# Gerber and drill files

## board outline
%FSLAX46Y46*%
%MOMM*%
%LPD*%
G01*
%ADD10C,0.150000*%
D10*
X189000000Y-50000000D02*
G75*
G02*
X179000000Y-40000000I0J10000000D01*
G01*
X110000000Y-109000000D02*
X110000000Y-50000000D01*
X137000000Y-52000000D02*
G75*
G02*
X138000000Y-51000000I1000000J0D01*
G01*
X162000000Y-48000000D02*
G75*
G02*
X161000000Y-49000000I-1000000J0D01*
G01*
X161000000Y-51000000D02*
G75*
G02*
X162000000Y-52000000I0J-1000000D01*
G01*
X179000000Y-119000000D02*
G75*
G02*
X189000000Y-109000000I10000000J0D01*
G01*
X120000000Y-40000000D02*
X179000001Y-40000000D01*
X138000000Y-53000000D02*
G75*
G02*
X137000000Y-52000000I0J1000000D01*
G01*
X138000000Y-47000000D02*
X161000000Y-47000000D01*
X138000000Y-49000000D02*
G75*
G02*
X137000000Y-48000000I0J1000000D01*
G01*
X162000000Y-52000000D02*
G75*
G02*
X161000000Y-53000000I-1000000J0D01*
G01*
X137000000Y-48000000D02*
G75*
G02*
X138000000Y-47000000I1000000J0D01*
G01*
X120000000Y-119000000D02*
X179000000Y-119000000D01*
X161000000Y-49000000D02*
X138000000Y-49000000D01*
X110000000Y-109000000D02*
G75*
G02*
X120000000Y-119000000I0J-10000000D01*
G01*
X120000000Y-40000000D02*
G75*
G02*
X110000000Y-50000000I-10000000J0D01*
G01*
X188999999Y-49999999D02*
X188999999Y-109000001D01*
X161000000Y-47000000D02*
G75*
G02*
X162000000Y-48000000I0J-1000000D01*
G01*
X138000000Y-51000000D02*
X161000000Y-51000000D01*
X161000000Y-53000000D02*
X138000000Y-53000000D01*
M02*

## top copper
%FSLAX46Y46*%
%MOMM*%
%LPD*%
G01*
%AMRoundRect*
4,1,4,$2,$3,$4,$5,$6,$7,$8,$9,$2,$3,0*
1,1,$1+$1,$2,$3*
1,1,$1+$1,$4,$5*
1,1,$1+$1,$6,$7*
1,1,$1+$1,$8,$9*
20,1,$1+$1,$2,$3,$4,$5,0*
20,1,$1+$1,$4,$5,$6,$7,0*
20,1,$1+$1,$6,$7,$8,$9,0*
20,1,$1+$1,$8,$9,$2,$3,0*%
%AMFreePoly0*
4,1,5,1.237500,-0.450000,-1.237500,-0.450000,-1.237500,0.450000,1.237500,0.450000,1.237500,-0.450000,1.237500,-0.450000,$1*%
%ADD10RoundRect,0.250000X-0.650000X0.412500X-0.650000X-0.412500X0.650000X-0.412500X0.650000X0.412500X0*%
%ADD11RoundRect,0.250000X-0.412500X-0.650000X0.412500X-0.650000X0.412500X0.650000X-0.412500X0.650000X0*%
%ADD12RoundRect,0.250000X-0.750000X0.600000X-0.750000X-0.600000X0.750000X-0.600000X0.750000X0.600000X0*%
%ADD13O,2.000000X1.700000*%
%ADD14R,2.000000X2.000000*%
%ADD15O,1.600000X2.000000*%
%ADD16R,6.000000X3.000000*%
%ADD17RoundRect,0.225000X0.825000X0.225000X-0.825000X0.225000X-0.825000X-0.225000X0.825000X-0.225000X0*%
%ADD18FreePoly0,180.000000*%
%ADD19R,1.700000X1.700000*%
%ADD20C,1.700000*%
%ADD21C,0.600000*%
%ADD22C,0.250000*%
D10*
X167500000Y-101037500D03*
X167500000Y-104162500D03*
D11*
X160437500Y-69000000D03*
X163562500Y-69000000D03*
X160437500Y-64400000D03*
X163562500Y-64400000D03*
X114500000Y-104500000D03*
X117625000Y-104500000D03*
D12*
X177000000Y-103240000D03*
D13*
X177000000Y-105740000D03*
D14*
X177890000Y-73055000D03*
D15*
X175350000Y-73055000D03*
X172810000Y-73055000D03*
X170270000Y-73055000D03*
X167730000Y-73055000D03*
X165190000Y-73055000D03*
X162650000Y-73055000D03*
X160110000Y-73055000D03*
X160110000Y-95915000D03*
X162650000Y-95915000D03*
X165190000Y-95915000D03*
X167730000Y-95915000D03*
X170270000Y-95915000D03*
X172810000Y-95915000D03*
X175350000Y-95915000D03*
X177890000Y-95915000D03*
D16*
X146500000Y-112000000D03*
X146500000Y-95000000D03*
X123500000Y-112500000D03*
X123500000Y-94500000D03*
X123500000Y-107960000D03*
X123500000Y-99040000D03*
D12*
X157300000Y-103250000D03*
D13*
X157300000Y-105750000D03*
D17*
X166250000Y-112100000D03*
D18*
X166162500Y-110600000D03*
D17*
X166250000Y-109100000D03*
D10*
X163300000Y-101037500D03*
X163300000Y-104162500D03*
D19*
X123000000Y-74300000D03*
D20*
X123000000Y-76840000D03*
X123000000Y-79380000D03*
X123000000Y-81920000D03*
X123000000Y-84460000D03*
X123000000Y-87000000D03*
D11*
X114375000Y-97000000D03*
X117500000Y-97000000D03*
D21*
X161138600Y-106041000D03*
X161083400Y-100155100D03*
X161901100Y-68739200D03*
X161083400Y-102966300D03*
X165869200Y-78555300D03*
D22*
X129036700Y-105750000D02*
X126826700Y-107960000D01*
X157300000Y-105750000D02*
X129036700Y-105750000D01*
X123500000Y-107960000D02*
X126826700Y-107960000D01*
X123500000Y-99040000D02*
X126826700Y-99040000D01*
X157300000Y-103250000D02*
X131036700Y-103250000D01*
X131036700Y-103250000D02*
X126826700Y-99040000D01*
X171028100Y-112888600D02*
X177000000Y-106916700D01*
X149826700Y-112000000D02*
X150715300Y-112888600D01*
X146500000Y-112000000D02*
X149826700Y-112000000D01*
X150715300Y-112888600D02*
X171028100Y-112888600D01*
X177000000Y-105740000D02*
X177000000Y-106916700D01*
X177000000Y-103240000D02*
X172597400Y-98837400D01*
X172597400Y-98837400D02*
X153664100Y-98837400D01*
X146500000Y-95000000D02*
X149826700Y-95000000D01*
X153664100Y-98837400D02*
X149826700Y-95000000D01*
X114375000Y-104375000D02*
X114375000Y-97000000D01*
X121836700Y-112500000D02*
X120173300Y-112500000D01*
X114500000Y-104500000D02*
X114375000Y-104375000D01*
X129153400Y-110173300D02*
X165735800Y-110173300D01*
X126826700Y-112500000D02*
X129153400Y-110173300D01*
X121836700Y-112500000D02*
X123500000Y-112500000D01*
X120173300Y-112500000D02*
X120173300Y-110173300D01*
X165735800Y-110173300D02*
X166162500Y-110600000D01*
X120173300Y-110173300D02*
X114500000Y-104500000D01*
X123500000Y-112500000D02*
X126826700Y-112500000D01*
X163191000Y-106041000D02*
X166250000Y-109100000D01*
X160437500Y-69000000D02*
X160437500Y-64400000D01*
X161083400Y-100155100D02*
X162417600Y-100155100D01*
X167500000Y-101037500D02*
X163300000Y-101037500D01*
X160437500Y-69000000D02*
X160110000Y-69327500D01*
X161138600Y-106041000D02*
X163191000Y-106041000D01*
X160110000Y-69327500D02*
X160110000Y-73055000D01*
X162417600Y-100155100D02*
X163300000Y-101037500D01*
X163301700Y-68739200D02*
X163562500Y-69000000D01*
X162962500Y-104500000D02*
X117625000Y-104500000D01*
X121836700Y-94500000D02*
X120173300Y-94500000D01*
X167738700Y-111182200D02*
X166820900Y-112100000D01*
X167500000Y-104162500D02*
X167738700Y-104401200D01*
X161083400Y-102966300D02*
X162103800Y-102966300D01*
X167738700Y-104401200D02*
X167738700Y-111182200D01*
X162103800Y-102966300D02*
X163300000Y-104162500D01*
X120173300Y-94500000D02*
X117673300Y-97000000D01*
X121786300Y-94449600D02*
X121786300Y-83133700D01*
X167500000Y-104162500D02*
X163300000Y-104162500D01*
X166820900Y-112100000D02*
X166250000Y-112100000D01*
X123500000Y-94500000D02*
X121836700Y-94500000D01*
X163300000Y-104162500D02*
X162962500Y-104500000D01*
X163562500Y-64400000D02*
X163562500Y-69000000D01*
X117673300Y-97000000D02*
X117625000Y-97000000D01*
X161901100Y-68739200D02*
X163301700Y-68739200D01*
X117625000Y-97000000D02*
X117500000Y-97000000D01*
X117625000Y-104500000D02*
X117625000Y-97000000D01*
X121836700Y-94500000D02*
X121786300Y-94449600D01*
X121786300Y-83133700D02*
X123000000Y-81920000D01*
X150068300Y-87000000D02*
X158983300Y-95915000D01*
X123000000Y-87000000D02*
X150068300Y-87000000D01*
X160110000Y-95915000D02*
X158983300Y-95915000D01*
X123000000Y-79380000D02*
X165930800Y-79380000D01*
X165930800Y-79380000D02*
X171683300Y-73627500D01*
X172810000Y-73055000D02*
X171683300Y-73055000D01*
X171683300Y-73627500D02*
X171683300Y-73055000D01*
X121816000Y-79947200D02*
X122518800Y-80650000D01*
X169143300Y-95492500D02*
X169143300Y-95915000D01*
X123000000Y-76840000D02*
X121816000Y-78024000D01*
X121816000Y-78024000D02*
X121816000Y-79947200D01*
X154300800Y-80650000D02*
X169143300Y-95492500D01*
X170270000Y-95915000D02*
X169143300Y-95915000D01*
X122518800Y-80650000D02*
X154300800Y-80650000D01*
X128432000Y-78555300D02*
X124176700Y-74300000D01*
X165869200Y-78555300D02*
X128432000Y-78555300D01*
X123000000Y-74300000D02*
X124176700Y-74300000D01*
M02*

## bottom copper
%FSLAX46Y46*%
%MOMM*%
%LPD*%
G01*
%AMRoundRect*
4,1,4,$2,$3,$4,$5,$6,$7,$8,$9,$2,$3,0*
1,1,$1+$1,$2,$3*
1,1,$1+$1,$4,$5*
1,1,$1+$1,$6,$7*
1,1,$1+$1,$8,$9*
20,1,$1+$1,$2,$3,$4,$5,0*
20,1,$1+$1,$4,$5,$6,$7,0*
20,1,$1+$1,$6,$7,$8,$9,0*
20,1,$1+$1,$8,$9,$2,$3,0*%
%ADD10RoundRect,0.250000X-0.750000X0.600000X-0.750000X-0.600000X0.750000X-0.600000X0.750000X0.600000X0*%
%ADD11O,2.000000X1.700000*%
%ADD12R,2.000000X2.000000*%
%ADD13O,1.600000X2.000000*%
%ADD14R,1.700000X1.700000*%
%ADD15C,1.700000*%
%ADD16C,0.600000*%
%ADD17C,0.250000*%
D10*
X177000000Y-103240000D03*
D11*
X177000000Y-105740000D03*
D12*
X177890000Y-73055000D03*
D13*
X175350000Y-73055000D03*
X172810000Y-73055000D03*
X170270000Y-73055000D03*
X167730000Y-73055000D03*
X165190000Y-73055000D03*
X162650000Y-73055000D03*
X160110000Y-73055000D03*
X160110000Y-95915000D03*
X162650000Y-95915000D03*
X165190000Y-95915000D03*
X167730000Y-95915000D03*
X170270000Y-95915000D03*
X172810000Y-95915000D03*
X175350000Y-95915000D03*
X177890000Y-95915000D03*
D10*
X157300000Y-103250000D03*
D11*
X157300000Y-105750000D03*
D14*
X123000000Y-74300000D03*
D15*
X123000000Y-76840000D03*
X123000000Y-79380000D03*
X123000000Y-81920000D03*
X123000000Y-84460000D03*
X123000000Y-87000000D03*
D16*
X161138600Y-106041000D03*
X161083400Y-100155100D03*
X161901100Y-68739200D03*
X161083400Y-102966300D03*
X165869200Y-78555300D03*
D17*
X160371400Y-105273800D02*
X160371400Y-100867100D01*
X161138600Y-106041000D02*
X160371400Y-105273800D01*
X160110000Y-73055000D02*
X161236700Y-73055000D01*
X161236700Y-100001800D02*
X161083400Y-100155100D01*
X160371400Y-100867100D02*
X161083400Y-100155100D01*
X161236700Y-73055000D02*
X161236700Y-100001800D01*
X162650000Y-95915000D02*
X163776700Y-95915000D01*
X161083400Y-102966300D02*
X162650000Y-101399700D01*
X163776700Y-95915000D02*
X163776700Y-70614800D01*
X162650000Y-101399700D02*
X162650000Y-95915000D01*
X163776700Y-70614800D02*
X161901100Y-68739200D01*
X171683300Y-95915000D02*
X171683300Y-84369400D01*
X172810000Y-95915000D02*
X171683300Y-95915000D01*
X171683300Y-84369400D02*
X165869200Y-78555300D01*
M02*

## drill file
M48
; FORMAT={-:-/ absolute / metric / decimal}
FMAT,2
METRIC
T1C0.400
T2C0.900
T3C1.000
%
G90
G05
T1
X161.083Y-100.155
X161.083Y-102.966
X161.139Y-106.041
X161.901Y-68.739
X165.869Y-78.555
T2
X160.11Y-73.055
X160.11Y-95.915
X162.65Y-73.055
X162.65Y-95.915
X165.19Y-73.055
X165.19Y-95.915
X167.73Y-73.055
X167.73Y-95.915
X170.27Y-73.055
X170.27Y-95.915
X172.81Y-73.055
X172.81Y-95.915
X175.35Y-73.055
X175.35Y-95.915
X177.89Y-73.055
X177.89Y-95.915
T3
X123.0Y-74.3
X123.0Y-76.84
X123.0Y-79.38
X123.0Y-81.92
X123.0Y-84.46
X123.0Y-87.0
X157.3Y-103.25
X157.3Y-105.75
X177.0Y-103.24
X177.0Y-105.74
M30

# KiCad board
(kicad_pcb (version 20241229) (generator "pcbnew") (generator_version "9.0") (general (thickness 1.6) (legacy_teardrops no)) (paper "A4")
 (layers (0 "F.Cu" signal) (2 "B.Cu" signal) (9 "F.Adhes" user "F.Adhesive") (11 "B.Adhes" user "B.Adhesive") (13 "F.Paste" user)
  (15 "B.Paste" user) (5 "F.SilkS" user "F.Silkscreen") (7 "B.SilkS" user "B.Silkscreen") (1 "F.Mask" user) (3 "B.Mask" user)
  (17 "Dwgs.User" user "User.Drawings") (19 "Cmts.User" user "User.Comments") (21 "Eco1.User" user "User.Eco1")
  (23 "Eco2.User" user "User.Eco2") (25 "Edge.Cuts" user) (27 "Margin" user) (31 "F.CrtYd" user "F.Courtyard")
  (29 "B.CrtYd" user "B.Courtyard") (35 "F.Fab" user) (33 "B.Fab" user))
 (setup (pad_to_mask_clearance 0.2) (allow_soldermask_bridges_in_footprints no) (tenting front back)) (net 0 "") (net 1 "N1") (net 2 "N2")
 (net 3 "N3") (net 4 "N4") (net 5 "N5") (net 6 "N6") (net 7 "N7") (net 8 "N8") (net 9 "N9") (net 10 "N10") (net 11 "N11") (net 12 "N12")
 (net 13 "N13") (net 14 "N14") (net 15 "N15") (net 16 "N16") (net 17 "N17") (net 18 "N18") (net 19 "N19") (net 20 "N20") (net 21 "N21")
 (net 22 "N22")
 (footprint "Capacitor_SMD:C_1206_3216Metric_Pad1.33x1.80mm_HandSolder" (layer "F.Cu") (at 167.5 102.6 -90)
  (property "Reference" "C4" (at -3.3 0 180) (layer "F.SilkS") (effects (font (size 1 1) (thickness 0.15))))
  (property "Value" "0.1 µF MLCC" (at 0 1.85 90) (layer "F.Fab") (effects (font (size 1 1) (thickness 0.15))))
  (pad "1" smd roundrect (at -1.5625 0 270) (size 1.325 1.8) (layers "F.Cu" "F.Mask" "F.Paste") (roundrect_rratio 0.188679) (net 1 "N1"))
  (pad "2" smd roundrect (at 1.5625 0 270) (size 1.325 1.8) (layers "F.Cu" "F.Mask" "F.Paste") (roundrect_rratio 0.188679) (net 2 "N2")))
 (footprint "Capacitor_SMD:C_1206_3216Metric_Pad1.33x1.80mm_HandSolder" (layer "F.Cu") (at 162 69)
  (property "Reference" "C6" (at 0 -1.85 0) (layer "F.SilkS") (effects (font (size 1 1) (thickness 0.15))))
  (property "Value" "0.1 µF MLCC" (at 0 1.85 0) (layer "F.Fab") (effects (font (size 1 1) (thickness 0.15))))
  (pad "1" smd roundrect (at -1.5625 0) (size 1.325 1.8) (layers "F.Cu" "F.Mask" "F.Paste") (roundrect_rratio 0.188679) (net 1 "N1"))
  (pad "2" smd roundrect (at 1.5625 0) (size 1.325 1.8) (layers "F.Cu" "F.Mask" "F.Paste") (roundrect_rratio 0.188679) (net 2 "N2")))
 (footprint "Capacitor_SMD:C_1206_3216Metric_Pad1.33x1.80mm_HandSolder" (layer "F.Cu") (at 162 64.4)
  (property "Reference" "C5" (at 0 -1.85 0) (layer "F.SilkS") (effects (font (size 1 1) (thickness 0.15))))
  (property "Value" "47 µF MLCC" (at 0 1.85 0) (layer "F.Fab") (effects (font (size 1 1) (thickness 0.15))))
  (pad "1" smd roundrect (at -1.5625 0) (size 1.325 1.8) (layers "F.Cu" "F.Mask" "F.Paste") (roundrect_rratio 0.188679) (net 1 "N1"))
  (pad "2" smd roundrect (at 1.5625 0) (size 1.325 1.8) (layers "F.Cu" "F.Mask" "F.Paste") (roundrect_rratio 0.188679) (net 2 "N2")))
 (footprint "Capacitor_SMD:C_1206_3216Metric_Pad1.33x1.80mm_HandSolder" (layer "F.Cu") (at 116.0625 104.5)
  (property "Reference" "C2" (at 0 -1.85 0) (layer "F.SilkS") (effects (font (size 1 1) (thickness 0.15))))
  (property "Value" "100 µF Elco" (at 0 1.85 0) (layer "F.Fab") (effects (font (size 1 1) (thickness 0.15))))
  (pad "1" smd roundrect (at -1.5625 0) (size 1.325 1.8) (layers "F.Cu" "F.Mask" "F.Paste") (roundrect_rratio 0.188679) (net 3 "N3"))
  (pad "2" smd roundrect (at 1.5625 0) (size 1.325 1.8) (layers "F.Cu" "F.Mask" "F.Paste") (roundrect_rratio 0.188679) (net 2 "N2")))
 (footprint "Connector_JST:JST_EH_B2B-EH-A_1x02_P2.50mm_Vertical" (layer "F.Cu") (at 177 103.24 -90)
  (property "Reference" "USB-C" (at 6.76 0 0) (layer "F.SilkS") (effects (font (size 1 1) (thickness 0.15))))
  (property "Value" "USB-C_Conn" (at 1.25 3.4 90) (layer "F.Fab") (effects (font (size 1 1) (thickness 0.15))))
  (pad "1" thru_hole roundrect (at 0 0 270) (size 1.7 2) (drill 1) (layers "*.Cu" "*.Mask") (remove_unused_layers no)
   (roundrect_rratio 0.147059) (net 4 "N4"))
  (pad "2" thru_hole oval (at 2.5 0 270) (size 1.7 2) (drill 1) (layers "*.Cu" "*.Mask") (remove_unused_layers no) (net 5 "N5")))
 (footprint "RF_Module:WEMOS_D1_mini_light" (layer "F.Cu") (at 177.89 73.055 -90)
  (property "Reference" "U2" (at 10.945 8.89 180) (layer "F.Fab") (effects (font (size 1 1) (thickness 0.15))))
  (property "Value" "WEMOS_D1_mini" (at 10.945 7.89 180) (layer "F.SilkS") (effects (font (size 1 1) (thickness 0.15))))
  (pad "1" thru_hole rect (at 0 0 270) (size 2 2) (drill 0.9) (layers "*.Cu" "*.Mask") (remove_unused_layers no) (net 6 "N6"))
  (pad "2" thru_hole oval (at 0 2.54 270) (size 2 1.6) (drill 0.9) (layers "*.Cu" "*.Mask") (remove_unused_layers no) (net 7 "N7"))
  (pad "3" thru_hole oval (at 0 5.08 270) (size 2 1.6) (drill 0.9) (layers "*.Cu" "*.Mask") (remove_unused_layers no) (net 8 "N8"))
  (pad "4" thru_hole oval (at 0 7.62 270) (size 2 1.6) (drill 0.9) (layers "*.Cu" "*.Mask") (remove_unused_layers no) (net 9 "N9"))
  (pad "5" thru_hole oval (at 0 10.16 270) (size 2 1.6) (drill 0.9) (layers "*.Cu" "*.Mask") (remove_unused_layers no) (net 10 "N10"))
  (pad "6" thru_hole oval (at 0 12.7 270) (size 2 1.6) (drill 0.9) (layers "*.Cu" "*.Mask") (remove_unused_layers no) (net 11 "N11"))
  (pad "7" thru_hole oval (at 0 15.24 270) (size 2 1.6) (drill 0.9) (layers "*.Cu" "*.Mask") (remove_unused_layers no) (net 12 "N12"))
  (pad "8" thru_hole oval (at 0 17.78 270) (size 2 1.6) (drill 0.9) (layers "*.Cu" "*.Mask") (remove_unused_layers no) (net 1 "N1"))
  (pad "9" thru_hole oval (at 22.86 17.78 270) (size 2 1.6) (drill 0.9) (layers "*.Cu" "*.Mask") (remove_unused_layers no) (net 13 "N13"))
  (pad "10" thru_hole oval (at 22.86 15.24 270) (size 2 1.6) (drill 0.9) (layers "*.Cu" "*.Mask") (remove_unused_layers no) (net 2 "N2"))
  (pad "11" thru_hole oval (at 22.86 12.7 270) (size 2 1.6) (drill 0.9) (layers "*.Cu" "*.Mask") (remove_unused_layers no) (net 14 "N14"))
  (pad "12" thru_hole oval (at 22.86 10.16 270) (size 2 1.6) (drill 0.9) (layers "*.Cu" "*.Mask") (remove_unused_layers no) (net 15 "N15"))
  (pad "13" thru_hole oval (at 22.86 7.62 270) (size 2 1.6) (drill 0.9) (layers "*.Cu" "*.Mask") (remove_unused_layers no) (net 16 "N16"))
  (pad "14" thru_hole oval (at 22.86 5.08 270) (size 2 1.6) (drill 0.9) (layers "*.Cu" "*.Mask") (remove_unused_layers no) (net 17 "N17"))
  (pad "15" thru_hole oval (at 22.86 2.54 270) (size 2 1.6) (drill 0.9) (layers "*.Cu" "*.Mask") (remove_unused_layers no) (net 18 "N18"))
  (pad "16" thru_hole oval (at 22.86 0 270) (size 2 1.6) (drill 0.9) (layers "*.Cu" "*.Mask") (remove_unused_layers no) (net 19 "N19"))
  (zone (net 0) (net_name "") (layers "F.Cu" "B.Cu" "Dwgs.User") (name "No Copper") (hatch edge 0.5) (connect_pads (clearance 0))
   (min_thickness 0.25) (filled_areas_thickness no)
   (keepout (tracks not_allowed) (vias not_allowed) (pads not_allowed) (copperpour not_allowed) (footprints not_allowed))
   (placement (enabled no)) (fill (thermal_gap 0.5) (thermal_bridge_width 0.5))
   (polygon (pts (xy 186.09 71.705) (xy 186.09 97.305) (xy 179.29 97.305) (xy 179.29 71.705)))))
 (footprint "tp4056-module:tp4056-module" (layer "F.Cu") (at 149 94.9 180)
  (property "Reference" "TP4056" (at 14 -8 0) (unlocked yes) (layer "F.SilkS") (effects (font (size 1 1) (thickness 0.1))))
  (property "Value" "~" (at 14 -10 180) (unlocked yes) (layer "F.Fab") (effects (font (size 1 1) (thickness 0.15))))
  (pad "1" smd rect (at 2.5 -17.1 180) (size 6 3) (layers "F.Cu" "F.Mask" "F.Paste") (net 5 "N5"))
  (pad "2" smd rect (at 2.5 -0.1 180) (size 6 3) (layers "F.Cu" "F.Mask" "F.Paste") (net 4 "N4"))
  (pad "3" smd rect (at 25.5 -17.6 180) (size 6 3) (layers "F.Cu" "F.Mask" "F.Paste") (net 3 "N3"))
  (pad "4" smd rect (at 25.5 0.4 180) (size 6 3) (layers "F.Cu" "F.Mask" "F.Paste") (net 2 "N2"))
  (pad "5" smd rect (at 25.5 -13.06 180) (size 6 3) (layers "F.Cu" "F.Mask" "F.Paste") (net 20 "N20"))
  (pad "6" smd rect (at 25.5 -4.14 180) (size 6 3) (layers "F.Cu" "F.Mask" "F.Paste") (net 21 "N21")))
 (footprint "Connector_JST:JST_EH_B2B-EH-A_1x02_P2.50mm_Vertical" (layer "F.Cu") (at 157.3 103.25 -90)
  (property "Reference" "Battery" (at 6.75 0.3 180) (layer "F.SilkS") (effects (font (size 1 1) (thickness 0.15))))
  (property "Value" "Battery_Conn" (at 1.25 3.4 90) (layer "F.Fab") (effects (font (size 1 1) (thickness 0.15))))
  (pad "1" thru_hole roundrect (at 0 0 270) (size 1.7 2) (drill 1) (layers "*.Cu" "*.Mask") (remove_unused_layers no)
   (roundrect_rratio 0.147059) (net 21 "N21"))
  (pad "2" thru_hole oval (at 2.5 0 270) (size 1.7 2) (drill 1) (layers "*.Cu" "*.Mask") (remove_unused_layers no) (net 20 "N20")))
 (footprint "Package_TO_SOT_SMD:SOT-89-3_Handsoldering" (layer "F.Cu") (at 163.8 110.6 180)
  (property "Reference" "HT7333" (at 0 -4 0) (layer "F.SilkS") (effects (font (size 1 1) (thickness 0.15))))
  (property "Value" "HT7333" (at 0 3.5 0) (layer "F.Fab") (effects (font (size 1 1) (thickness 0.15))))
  (pad "1" smd roundrect (at -2.45 -1.5 180) (size 2.1 0.9) (layers "F.Cu" "F.Mask" "F.Paste") (roundrect_rratio 0.25) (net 2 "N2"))
  (pad "2" smd custom (at -2.3625 0 180) (size 2.475 0.9) (layers "F.Cu" "F.Mask" "F.Paste") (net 3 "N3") (zone_connect 2)
   (thermal_bridge_angle 45) (options (clearance outline) (anchor rect)) (primitives))
  (pad "3" smd roundrect (at -2.45 1.5 180) (size 2.1 0.9) (layers "F.Cu" "F.Mask" "F.Paste") (roundrect_rratio 0.25) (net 1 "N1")))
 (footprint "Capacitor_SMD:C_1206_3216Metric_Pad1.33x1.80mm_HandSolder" (layer "F.Cu") (at 163.3 102.6 -90)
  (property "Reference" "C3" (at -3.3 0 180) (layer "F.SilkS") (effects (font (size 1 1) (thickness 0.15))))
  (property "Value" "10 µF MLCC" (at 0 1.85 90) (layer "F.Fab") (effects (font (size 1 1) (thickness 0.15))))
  (pad "1" smd roundrect (at -1.5625 0 270) (size 1.325 1.8) (layers "F.Cu" "F.Mask" "F.Paste") (roundrect_rratio 0.188679) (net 1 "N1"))
  (pad "2" smd roundrect (at 1.5625 0 270) (size 1.325 1.8) (layers "F.Cu" "F.Mask" "F.Paste") (roundrect_rratio 0.188679) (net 2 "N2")))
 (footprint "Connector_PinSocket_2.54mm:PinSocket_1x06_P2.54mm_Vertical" (layer "F.Cu") (at 123 74.3)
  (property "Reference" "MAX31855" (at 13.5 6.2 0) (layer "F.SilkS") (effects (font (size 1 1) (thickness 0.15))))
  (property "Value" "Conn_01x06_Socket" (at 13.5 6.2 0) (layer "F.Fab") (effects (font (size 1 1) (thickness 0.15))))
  (pad "1" thru_hole rect (at 0 0) (size 1.7 1.7) (drill 1) (layers "*.Cu" "*.Mask") (remove_unused_layers no) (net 17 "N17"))
  (pad "2" thru_hole circle (at 0 2.54) (size 1.7 1.7) (drill 1) (layers "*.Cu" "*.Mask") (remove_unused_layers no) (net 16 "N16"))
  (pad "3" thru_hole circle (at 0 5.08) (size 1.7 1.7) (drill 1) (layers "*.Cu" "*.Mask") (remove_unused_layers no) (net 8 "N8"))
  (pad "4" thru_hole circle (at 0 7.62) (size 1.7 1.7) (drill 1) (layers "*.Cu" "*.Mask") (remove_unused_layers no) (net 2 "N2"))
  (pad "5" thru_hole circle (at 0 10.16) (size 1.7 1.7) (drill 1) (layers "*.Cu" "*.Mask") (remove_unused_layers no) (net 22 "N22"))
  (pad "6" thru_hole circle (at 0 12.7) (size 1.7 1.7) (drill 1) (layers "*.Cu" "*.Mask") (remove_unused_layers no) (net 13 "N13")))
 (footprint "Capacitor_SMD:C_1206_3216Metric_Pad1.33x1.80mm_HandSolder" (layer "F.Cu") (at 115.9375 97)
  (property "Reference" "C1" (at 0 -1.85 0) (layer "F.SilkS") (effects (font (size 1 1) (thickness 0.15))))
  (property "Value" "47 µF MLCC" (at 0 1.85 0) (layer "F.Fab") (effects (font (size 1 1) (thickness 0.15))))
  (pad "1" smd roundrect (at -1.5625 0) (size 1.325 1.8) (layers "F.Cu" "F.Mask" "F.Paste") (roundrect_rratio 0.188679) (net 3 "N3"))
  (pad "2" smd roundrect (at 1.5625 0) (size 1.325 1.8) (layers "F.Cu" "F.Mask" "F.Paste") (roundrect_rratio 0.188679) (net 2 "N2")))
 (gr_arc (start 189 50) (mid 181.928932 47.071068) (end 179.000001 40) (stroke (width 0.15) (type solid)) (layer "Edge.Cuts"))
 (gr_line (start 110 109) (end 110 50) (stroke (width 0.15) (type solid)) (layer "Edge.Cuts"))
 (gr_arc (start 137 52) (mid 137.292893 51.292893) (end 138 51) (stroke (width 0.15) (type default)) (layer "Edge.Cuts"))
 (gr_arc (start 162 48) (mid 161.707107 48.707107) (end 161 49) (stroke (width 0.15) (type default)) (layer "Edge.Cuts"))
 (gr_arc (start 161 51) (mid 161.707107 51.292893) (end 162 52) (stroke (width 0.15) (type default)) (layer "Edge.Cuts"))
 (gr_arc (start 179 119) (mid 181.928932 111.928932) (end 189 109) (stroke (width 0.15) (type solid)) (layer "Edge.Cuts"))
 (gr_line (start 120 40) (end 179.000001 40) (stroke (width 0.15) (type solid)) (layer "Edge.Cuts"))
 (gr_arc (start 138 53) (mid 137.292893 52.707107) (end 137 52) (stroke (width 0.15) (type default)) (layer "Edge.Cuts"))
 (gr_line (start 138 47) (end 161 47) (stroke (width 0.15) (type default)) (layer "Edge.Cuts"))
 (gr_arc (start 138 49) (mid 137.292893 48.707107) (end 137 48) (stroke (width 0.15) (type default)) (layer "Edge.Cuts"))
 (gr_arc (start 162 52) (mid 161.707107 52.707107) (end 161 53) (stroke (width 0.15) (type default)) (layer "Edge.Cuts"))
 (gr_arc (start 137 48) (mid 137.292893 47.292893) (end 138 47) (stroke (width 0.15) (type default)) (layer "Edge.Cuts"))
 (gr_line (start 120 119) (end 179 119) (stroke (width 0.15) (type solid)) (layer "Edge.Cuts"))
 (gr_line (start 161 49) (end 138 49) (stroke (width 0.15) (type default)) (layer "Edge.Cuts"))
 (gr_arc (start 110 109) (mid 117.071068 111.928932) (end 120 119) (stroke (width 0.15) (type solid)) (layer "Edge.Cuts"))
 (gr_arc (start 120 40) (mid 117.071068 47.071068) (end 110 50) (stroke (width 0.15) (type solid)) (layer "Edge.Cuts"))
 (gr_line (start 188.999999 49.999999) (end 188.999999 109.000001) (stroke (width 0.15) (type solid)) (layer "Edge.Cuts"))
 (gr_arc (start 161 47) (mid 161.707107 47.292893) (end 162 48) (stroke (width 0.15) (type default)) (layer "Edge.Cuts"))
 (gr_line (start 138 51) (end 161 51) (stroke (width 0.15) (type default)) (layer "Edge.Cuts"))
 (gr_line (start 161 53) (end 138 53) (stroke (width 0.15) (type default)) (layer "Edge.Cuts"))
 (segment (start 129.0367 105.75) (end 126.8267 107.96) (width 0.25) (layer "F.Cu") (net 20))
 (segment (start 157.3 105.75) (end 129.0367 105.75) (width 0.25) (layer "F.Cu") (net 20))
 (segment (start 123.5 107.96) (end 126.8267 107.96) (width 0.25) (layer "F.Cu") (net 20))
 (segment (start 123.5 99.04) (end 126.8267 99.04) (width 0.25) (layer "F.Cu") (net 21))
 (segment (start 157.3 103.25) (end 131.0367 103.25) (width 0.25) (layer "F.Cu") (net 21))
 (segment (start 131.0367 103.25) (end 126.8267 99.04) (width 0.25) (layer "F.Cu") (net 21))
 (segment (start 171.0281 112.8886) (end 177 106.9167) (width 0.25) (layer "F.Cu") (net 5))
 (segment (start 149.8267 112) (end 150.7153 112.8886) (width 0.25) (layer "F.Cu") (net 5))
 (segment (start 146.5 112) (end 149.8267 112) (width 0.25) (layer "F.Cu") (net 5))
 (segment (start 150.7153 112.8886) (end 171.0281 112.8886) (width 0.25) (layer "F.Cu") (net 5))
 (segment (start 177 105.74) (end 177 106.9167) (width 0.25) (layer "F.Cu") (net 5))
 (segment (start 177 103.24) (end 172.5974 98.8374) (width 0.25) (layer "F.Cu") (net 4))
 (segment (start 172.5974 98.8374) (end 153.6641 98.8374) (width 0.25) (layer "F.Cu") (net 4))
 (segment (start 146.5 95) (end 149.8267 95) (width 0.25) (layer "F.Cu") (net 4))
 (segment (start 153.6641 98.8374) (end 149.8267 95) (width 0.25) (layer "F.Cu") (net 4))
 (segment (start 114.375 104.375) (end 114.375 97) (width 0.25) (layer "F.Cu") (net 3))
 (segment (start 121.8367 112.5) (end 120.1733 112.5) (width 0.25) (layer "F.Cu") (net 3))
 (segment (start 114.5 104.5) (end 114.375 104.375) (width 0.25) (layer "F.Cu") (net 3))
 (segment (start 129.1534 110.1733) (end 165.7358 110.1733) (width 0.25) (layer "F.Cu") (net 3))
 (segment (start 126.8267 112.5) (end 129.1534 110.1733) (width 0.25) (layer "F.Cu") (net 3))
 (segment (start 121.8367 112.5) (end 123.5 112.5) (width 0.25) (layer "F.Cu") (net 3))
 (segment (start 120.1733 112.5) (end 120.1733 110.1733) (width 0.25) (layer "F.Cu") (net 3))
 (segment (start 165.7358 110.1733) (end 166.1625 110.6) (width 0.25) (layer "F.Cu") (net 3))
 (segment (start 120.1733 110.1733) (end 114.5 104.5) (width 0.25) (layer "F.Cu") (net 3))
 (segment (start 123.5 112.5) (end 126.8267 112.5) (width 0.25) (layer "F.Cu") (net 3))
 (segment (start 163.191 106.041) (end 166.25 109.1) (width 0.25) (layer "F.Cu") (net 1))
 (segment (start 160.4375 69) (end 160.4375 64.4) (width 0.25) (layer "F.Cu") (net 1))
 (segment (start 161.0834 100.1551) (end 162.4176 100.1551) (width 0.25) (layer "F.Cu") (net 1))
 (segment (start 167.5 101.0375) (end 163.3 101.0375) (width 0.25) (layer "F.Cu") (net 1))
 (segment (start 160.4375 69) (end 160.11 69.3275) (width 0.25) (layer "F.Cu") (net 1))
 (segment (start 161.1386 106.041) (end 163.191 106.041) (width 0.25) (layer "F.Cu") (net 1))
 (segment (start 160.11 69.3275) (end 160.11 73.055) (width 0.25) (layer "F.Cu") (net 1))
 (segment (start 162.4176 100.1551) (end 163.3 101.0375) (width 0.25) (layer "F.Cu") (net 1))
 (via (at 161.1386 106.041) (size 0.6) (drill 0.4) (layers "F.Cu" "B.Cu") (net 1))
 (via (at 161.0834 100.1551) (size 0.6) (drill 0.4) (layers "F.Cu" "B.Cu") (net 1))
 (segment (start 160.3714 105.2738) (end 160.3714 100.8671) (width 0.25) (layer "B.Cu") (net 1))
 (segment (start 161.1386 106.041) (end 160.3714 105.2738) (width 0.25) (layer "B.Cu") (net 1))
 (segment (start 160.11 73.055) (end 161.2367 73.055) (width 0.25) (layer "B.Cu") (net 1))
 (segment (start 161.2367 100.0018) (end 161.0834 100.1551) (width 0.25) (layer "B.Cu") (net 1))
 (segment (start 160.3714 100.8671) (end 161.0834 100.1551) (width 0.25) (layer "B.Cu") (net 1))
 (segment (start 161.2367 73.055) (end 161.2367 100.0018) (width 0.25) (layer "B.Cu") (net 1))
 (segment (start 163.3017 68.7392) (end 163.5625 69) (width 0.25) (layer "F.Cu") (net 2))
 (segment (start 162.9625 104.5) (end 117.625 104.5) (width 0.25) (layer "F.Cu") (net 2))
 (segment (start 121.8367 94.5) (end 120.1733 94.5) (width 0.25) (layer "F.Cu") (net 2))
 (segment (start 167.7387 111.1822) (end 166.8209 112.1) (width 0.25) (layer "F.Cu") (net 2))
 (segment (start 167.5 104.1625) (end 167.7387 104.4012) (width 0.25) (layer "F.Cu") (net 2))
 (segment (start 161.0834 102.9663) (end 162.1038 102.9663) (width 0.25) (layer "F.Cu") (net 2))
 (segment (start 167.7387 104.4012) (end 167.7387 111.1822) (width 0.25) (layer "F.Cu") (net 2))
 (segment (start 162.1038 102.9663) (end 163.3 104.1625) (width 0.25) (layer "F.Cu") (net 2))
 (segment (start 120.1733 94.5) (end 117.6733 97) (width 0.25) (layer "F.Cu") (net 2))
 (segment (start 121.7863 94.4496) (end 121.7863 83.1337) (width 0.25) (layer "F.Cu") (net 2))
 (segment (start 167.5 104.1625) (end 163.3 104.1625) (width 0.25) (layer "F.Cu") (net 2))
 (segment (start 166.8209 112.1) (end 166.25 112.1) (width 0.25) (layer "F.Cu") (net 2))
 (segment (start 123.5 94.5) (end 121.8367 94.5) (width 0.25) (layer "F.Cu") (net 2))
 (segment (start 163.3 104.1625) (end 162.9625 104.5) (width 0.25) (layer "F.Cu") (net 2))
 (segment (start 163.5625 64.4) (end 163.5625 69) (width 0.25) (layer "F.Cu") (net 2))
 (segment (start 117.6733 97) (end 117.625 97) (width 0.25) (layer "F.Cu") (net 2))
 (segment (start 161.9011 68.7392) (end 163.3017 68.7392) (width 0.25) (layer "F.Cu") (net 2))
 (segment (start 117.625 97) (end 117.5 97) (width 0.25) (layer "F.Cu") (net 2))
 (segment (start 117.625 104.5) (end 117.625 97) (width 0.25) (layer "F.Cu") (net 2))
 (segment (start 121.8367 94.5) (end 121.7863 94.4496) (width 0.25) (layer "F.Cu") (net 2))
 (segment (start 121.7863 83.1337) (end 123 81.92) (width 0.25) (layer "F.Cu") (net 2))
 (via (at 161.9011 68.7392) (size 0.6) (drill 0.4) (layers "F.Cu" "B.Cu") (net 2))
 (via (at 161.0834 102.9663) (size 0.6) (drill 0.4) (layers "F.Cu" "B.Cu") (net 2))
 (segment (start 162.65 95.915) (end 163.7767 95.915) (width 0.25) (layer "B.Cu") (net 2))
 (segment (start 161.0834 102.9663) (end 162.65 101.3997) (width 0.25) (layer "B.Cu") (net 2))
 (segment (start 163.7767 95.915) (end 163.7767 70.6148) (width 0.25) (layer "B.Cu") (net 2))
 (segment (start 162.65 101.3997) (end 162.65 95.915) (width 0.25) (layer "B.Cu") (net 2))
 (segment (start 163.7767 70.6148) (end 161.9011 68.7392) (width 0.25) (layer "B.Cu") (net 2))
 (segment (start 150.0683 87) (end 158.9833 95.915) (width 0.25) (layer "F.Cu") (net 13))
 (segment (start 123 87) (end 150.0683 87) (width 0.25) (layer "F.Cu") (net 13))
 (segment (start 160.11 95.915) (end 158.9833 95.915) (width 0.25) (layer "F.Cu") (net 13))
 (segment (start 123 79.38) (end 165.9308 79.38) (width 0.25) (layer "F.Cu") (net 8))
 (segment (start 165.9308 79.38) (end 171.6833 73.6275) (width 0.25) (layer "F.Cu") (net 8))
 (segment (start 172.81 73.055) (end 171.6833 73.055) (width 0.25) (layer "F.Cu") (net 8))
 (segment (start 171.6833 73.6275) (end 171.6833 73.055) (width 0.25) (layer "F.Cu") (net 8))
 (segment (start 121.816 79.9472) (end 122.5188 80.65) (width 0.25) (layer "F.Cu") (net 16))
 (segment (start 169.1433 95.4925) (end 169.1433 95.915) (width 0.25) (layer "F.Cu") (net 16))
 (segment (start 123 76.84) (end 121.816 78.024) (width 0.25) (layer "F.Cu") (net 16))
 (segment (start 121.816 78.024) (end 121.816 79.9472) (width 0.25) (layer "F.Cu") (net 16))
 (segment (start 154.3008 80.65) (end 169.1433 95.4925) (width 0.25) (layer "F.Cu") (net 16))
 (segment (start 170.27 95.915) (end 169.1433 95.915) (width 0.25) (layer "F.Cu") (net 16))
 (segment (start 122.5188 80.65) (end 154.3008 80.65) (width 0.25) (layer "F.Cu") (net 16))
 (segment (start 128.432 78.5553) (end 124.1767 74.3) (width 0.25) (layer "F.Cu") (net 17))
 (segment (start 165.8692 78.5553) (end 128.432 78.5553) (width 0.25) (layer "F.Cu") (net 17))
 (segment (start 123 74.3) (end 124.1767 74.3) (width 0.25) (layer "F.Cu") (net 17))
 (via (at 165.8692 78.5553) (size 0.6) (drill 0.4) (layers "F.Cu" "B.Cu") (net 17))
 (segment (start 171.6833 95.915) (end 171.6833 84.3694) (width 0.25) (layer "B.Cu") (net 17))
 (segment (start 172.81 95.915) (end 171.6833 95.915) (width 0.25) (layer "B.Cu") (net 17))
 (segment (start 171.6833 84.3694) (end 165.8692 78.5553) (width 0.25) (layer "B.Cu") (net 17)))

